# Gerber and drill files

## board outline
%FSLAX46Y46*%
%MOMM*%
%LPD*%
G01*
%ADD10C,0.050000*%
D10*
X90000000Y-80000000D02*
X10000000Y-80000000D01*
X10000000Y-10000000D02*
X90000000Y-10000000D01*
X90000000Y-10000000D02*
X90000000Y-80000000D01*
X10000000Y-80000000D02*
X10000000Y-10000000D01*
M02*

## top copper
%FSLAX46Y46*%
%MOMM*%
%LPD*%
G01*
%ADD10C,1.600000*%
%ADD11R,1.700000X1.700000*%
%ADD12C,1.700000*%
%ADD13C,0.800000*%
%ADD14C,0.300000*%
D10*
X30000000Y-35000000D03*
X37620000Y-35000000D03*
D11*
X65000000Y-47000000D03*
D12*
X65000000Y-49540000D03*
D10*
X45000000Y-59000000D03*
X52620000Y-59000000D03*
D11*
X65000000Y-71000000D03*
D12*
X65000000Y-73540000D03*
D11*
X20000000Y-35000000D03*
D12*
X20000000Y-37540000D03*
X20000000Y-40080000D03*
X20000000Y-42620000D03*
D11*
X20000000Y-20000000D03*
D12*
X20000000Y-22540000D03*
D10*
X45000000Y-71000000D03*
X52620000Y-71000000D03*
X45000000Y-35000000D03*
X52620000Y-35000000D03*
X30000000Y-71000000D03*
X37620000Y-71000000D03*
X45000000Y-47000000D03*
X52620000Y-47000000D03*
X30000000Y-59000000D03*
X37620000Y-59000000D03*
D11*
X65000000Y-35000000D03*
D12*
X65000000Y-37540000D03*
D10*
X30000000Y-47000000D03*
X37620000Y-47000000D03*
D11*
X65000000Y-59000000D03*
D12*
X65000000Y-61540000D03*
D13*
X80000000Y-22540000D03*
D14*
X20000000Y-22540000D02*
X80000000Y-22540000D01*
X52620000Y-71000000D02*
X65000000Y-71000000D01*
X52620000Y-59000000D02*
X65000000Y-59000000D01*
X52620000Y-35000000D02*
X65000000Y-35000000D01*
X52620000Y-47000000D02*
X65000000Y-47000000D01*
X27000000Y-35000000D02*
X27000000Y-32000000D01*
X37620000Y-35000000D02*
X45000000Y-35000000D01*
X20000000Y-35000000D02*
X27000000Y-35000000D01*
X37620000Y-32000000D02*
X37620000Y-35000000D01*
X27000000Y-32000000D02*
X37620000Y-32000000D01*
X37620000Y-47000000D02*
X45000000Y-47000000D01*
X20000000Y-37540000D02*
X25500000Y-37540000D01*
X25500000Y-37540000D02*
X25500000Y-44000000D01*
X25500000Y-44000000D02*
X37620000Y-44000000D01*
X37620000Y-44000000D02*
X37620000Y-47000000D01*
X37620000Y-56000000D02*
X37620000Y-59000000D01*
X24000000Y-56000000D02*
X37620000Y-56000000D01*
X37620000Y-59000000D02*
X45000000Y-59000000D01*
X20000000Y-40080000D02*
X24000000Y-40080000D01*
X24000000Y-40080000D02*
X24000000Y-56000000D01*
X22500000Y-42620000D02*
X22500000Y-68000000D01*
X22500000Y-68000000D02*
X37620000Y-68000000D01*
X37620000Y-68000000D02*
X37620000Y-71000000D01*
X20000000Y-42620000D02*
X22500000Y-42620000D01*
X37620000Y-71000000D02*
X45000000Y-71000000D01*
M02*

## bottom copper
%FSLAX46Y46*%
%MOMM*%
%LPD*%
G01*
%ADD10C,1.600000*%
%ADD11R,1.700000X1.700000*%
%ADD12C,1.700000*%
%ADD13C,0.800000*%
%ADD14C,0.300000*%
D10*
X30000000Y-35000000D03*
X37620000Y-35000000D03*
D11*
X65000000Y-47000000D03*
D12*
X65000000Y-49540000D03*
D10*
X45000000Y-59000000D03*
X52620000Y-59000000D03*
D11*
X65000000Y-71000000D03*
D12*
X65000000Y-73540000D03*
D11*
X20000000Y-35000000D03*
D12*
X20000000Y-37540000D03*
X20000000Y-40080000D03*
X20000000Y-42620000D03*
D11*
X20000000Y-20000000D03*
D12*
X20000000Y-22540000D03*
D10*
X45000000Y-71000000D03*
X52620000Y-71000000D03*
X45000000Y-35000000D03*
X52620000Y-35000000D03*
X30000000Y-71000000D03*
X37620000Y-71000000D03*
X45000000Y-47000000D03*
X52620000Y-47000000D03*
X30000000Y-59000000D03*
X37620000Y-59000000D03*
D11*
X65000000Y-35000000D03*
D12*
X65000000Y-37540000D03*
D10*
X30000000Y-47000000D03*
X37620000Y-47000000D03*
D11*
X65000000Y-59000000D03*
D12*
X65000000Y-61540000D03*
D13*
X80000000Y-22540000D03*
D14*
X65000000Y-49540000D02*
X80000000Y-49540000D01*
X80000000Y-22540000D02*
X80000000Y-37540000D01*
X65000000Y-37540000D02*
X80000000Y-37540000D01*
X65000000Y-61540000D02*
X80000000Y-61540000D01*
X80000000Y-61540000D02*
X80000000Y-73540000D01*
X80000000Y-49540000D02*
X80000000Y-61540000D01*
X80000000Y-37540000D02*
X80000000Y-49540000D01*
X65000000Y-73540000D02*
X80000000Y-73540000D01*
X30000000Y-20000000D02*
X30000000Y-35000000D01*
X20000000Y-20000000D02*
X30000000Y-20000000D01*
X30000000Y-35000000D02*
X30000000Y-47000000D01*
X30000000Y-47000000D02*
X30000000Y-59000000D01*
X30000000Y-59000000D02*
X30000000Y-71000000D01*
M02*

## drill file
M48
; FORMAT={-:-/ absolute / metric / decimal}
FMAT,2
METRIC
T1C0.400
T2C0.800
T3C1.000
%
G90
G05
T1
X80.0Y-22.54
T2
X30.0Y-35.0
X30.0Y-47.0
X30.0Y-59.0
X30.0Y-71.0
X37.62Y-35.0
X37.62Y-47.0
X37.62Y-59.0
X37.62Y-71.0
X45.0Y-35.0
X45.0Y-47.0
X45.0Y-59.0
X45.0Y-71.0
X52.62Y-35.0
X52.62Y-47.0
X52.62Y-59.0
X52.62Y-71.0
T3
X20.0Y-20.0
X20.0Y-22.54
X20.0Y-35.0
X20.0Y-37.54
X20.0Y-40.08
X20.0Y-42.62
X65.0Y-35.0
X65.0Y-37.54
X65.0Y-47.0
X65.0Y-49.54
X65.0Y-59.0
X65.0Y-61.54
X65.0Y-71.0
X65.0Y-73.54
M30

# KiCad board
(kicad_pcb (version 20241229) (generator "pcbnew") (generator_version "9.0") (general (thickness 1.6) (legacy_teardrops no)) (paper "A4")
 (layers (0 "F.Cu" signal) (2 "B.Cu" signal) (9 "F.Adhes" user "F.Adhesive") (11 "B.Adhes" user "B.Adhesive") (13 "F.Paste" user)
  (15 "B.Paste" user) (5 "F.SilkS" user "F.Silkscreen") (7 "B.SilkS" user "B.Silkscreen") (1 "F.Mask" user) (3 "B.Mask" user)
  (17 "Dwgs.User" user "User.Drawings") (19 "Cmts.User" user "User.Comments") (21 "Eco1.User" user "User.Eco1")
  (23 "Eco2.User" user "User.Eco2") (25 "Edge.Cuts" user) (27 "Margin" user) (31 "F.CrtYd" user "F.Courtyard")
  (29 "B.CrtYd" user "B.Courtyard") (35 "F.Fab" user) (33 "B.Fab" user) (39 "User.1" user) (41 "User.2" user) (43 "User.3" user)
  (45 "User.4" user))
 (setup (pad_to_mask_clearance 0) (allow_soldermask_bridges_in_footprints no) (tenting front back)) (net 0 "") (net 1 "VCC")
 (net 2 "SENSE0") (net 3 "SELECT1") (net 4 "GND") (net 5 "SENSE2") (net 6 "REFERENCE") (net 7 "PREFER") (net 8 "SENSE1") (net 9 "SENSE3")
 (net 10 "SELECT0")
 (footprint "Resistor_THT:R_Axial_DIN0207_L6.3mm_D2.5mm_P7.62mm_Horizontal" (layer "F.Cu") (at 30 35)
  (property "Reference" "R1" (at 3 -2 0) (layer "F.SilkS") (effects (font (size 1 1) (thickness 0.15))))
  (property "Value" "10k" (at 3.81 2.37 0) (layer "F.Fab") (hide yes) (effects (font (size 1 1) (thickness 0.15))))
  (pad "1" thru_hole circle (at 0 0) (size 1.6 1.6) (drill 0.8) (layers "*.Cu" "*.Mask") (remove_unused_layers no) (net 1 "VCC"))
  (pad "2" thru_hole circle (at 7.62 0) (size 1.6 1.6) (drill 0.8) (layers "*.Cu" "*.Mask") (remove_unused_layers no) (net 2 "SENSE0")))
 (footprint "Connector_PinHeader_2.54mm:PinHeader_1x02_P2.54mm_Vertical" (layer "F.Cu") (at 65 47)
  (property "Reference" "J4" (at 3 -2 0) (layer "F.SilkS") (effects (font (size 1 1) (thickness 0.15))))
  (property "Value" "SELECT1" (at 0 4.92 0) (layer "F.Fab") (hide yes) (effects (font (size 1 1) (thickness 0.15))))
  (pad "1" thru_hole rect (at 0 0) (size 1.7 1.7) (drill 1) (layers "*.Cu" "*.Mask") (remove_unused_layers no) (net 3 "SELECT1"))
  (pad "2" thru_hole circle (at 0 2.54) (size 1.7 1.7) (drill 1) (layers "*.Cu" "*.Mask") (remove_unused_layers no) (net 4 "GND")))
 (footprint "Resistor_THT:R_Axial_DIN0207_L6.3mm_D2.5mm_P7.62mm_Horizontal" (layer "F.Cu") (at 45 59)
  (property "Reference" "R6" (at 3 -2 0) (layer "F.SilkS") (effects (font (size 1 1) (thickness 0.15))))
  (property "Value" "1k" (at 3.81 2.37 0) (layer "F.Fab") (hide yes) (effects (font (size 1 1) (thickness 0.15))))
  (pad "1" thru_hole circle (at 0 0) (size 1.6 1.6) (drill 0.8) (layers "*.Cu" "*.Mask") (remove_unused_layers no) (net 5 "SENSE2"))
  (pad "2" thru_hole circle (at 7.62 0) (size 1.6 1.6) (drill 0.8) (layers "*.Cu" "*.Mask") (remove_unused_layers no) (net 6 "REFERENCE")))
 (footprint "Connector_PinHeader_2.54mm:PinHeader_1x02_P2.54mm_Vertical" (layer "F.Cu") (at 65 71)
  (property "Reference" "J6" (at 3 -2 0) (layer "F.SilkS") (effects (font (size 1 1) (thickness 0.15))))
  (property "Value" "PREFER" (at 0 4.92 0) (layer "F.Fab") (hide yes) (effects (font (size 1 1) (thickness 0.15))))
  (pad "1" thru_hole rect (at 0 0) (size 1.7 1.7) (drill 1) (layers "*.Cu" "*.Mask") (remove_unused_layers no) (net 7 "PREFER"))
  (pad "2" thru_hole circle (at 0 2.54) (size 1.7 1.7) (drill 1) (layers "*.Cu" "*.Mask") (remove_unused_layers no) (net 4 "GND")))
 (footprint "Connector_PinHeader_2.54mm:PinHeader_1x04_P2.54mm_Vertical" (layer "F.Cu") (at 20 35)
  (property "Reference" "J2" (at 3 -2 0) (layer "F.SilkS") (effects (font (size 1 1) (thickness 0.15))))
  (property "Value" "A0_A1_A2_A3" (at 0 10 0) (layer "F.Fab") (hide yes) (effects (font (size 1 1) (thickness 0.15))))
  (pad "1" thru_hole rect (at 0 0) (size 1.7 1.7) (drill 1) (layers "*.Cu" "*.Mask") (remove_unused_layers no) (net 2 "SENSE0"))
  (pad "2" thru_hole circle (at 0 2.54) (size 1.7 1.7) (drill 1) (layers "*.Cu" "*.Mask") (remove_unused_layers no) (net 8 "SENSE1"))
  (pad "3" thru_hole circle (at 0 5.08) (size 1.7 1.7) (drill 1) (layers "*.Cu" "*.Mask") (remove_unused_layers no) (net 5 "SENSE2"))
  (pad "4" thru_hole circle (at 0 7.62) (size 1.7 1.7) (drill 1) (layers "*.Cu" "*.Mask") (remove_unused_layers no) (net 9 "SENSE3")))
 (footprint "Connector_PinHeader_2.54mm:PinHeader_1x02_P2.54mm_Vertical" (layer "F.Cu") (at 20 20)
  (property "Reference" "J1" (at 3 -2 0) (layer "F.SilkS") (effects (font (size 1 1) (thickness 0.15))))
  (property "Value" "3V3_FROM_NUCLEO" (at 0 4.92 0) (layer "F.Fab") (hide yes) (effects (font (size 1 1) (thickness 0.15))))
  (pad "1" thru_hole rect (at 0 0) (size 1.7 1.7) (drill 1) (layers "*.Cu" "*.Mask") (remove_unused_layers no) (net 1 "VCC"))
  (pad "2" thru_hole circle (at 0 2.54) (size 1.7 1.7) (drill 1) (layers "*.Cu" "*.Mask") (remove_unused_layers no) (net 4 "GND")))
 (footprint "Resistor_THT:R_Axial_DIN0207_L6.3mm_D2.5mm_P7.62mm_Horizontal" (layer "F.Cu") (at 45 71)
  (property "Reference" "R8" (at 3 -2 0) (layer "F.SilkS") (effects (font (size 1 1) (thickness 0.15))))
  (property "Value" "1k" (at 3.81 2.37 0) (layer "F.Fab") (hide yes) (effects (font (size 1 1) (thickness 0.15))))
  (pad "1" thru_hole circle (at 0 0) (size 1.6 1.6) (drill 0.8) (layers "*.Cu" "*.Mask") (remove_unused_layers no) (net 9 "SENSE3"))
  (pad "2" thru_hole circle (at 7.62 0) (size 1.6 1.6) (drill 0.8) (layers "*.Cu" "*.Mask") (remove_unused_layers no) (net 7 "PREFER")))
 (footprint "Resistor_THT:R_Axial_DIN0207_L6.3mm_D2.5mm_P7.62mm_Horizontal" (layer "F.Cu") (at 45 35)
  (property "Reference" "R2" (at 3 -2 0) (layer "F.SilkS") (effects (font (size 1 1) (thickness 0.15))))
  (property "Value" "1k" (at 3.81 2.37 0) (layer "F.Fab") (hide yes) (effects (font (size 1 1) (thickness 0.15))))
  (pad "1" thru_hole circle (at 0 0) (size 1.6 1.6) (drill 0.8) (layers "*.Cu" "*.Mask") (remove_unused_layers no) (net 2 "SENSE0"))
  (pad "2" thru_hole circle (at 7.62 0) (size 1.6 1.6) (drill 0.8) (layers "*.Cu" "*.Mask") (remove_unused_layers no) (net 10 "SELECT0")))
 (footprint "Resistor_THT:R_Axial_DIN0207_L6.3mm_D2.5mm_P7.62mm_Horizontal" (layer "F.Cu") (at 30 71)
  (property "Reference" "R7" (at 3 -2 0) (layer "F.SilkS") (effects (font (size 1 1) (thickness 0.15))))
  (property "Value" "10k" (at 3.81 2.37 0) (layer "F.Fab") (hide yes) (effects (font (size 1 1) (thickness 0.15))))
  (pad "1" thru_hole circle (at 0 0) (size 1.6 1.6) (drill 0.8) (layers "*.Cu" "*.Mask") (remove_unused_layers no) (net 1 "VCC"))
  (pad "2" thru_hole circle (at 7.62 0) (size 1.6 1.6) (drill 0.8) (layers "*.Cu" "*.Mask") (remove_unused_layers no) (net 9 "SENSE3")))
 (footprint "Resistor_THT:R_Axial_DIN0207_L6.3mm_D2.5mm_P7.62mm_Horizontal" (layer "F.Cu") (at 45 47)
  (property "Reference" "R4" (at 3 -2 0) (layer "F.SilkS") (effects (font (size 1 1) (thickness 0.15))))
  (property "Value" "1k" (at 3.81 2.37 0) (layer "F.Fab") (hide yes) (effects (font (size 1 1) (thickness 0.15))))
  (pad "1" thru_hole circle (at 0 0) (size 1.6 1.6) (drill 0.8) (layers "*.Cu" "*.Mask") (remove_unused_layers no) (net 8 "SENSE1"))
  (pad "2" thru_hole circle (at 7.62 0) (size 1.6 1.6) (drill 0.8) (layers "*.Cu" "*.Mask") (remove_unused_layers no) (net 3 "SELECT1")))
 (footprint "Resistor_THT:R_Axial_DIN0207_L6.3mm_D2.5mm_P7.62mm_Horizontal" (layer "F.Cu") (at 30 59)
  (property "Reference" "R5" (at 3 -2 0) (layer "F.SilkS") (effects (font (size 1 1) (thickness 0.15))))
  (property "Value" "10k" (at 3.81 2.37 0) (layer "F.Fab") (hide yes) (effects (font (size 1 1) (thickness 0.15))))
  (pad "1" thru_hole circle (at 0 0) (size 1.6 1.6) (drill 0.8) (layers "*.Cu" "*.Mask") (remove_unused_layers no) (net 1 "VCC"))
  (pad "2" thru_hole circle (at 7.62 0) (size 1.6 1.6) (drill 0.8) (layers "*.Cu" "*.Mask") (remove_unused_layers no) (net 5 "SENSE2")))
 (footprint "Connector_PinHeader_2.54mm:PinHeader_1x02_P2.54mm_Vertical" (layer "F.Cu") (at 65 35)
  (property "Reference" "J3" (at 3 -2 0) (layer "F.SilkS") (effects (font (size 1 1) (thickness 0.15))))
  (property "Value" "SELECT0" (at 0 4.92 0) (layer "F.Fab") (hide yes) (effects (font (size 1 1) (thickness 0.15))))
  (pad "1" thru_hole rect (at 0 0) (size 1.7 1.7) (drill 1) (layers "*.Cu" "*.Mask") (remove_unused_layers no) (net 10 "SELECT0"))
  (pad "2" thru_hole circle (at 0 2.54) (size 1.7 1.7) (drill 1) (layers "*.Cu" "*.Mask") (remove_unused_layers no) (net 4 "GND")))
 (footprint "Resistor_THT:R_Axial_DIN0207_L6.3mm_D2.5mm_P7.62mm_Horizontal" (layer "F.Cu") (at 30 47)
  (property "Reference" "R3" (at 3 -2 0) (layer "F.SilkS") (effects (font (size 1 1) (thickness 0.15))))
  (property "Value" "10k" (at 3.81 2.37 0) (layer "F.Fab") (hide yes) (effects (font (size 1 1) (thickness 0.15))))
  (pad "1" thru_hole circle (at 0 0) (size 1.6 1.6) (drill 0.8) (layers "*.Cu" "*.Mask") (remove_unused_layers no) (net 1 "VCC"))
  (pad "2" thru_hole circle (at 7.62 0) (size 1.6 1.6) (drill 0.8) (layers "*.Cu" "*.Mask") (remove_unused_layers no) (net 8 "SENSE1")))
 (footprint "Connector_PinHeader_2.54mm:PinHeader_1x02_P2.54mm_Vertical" (layer "F.Cu") (at 65 59)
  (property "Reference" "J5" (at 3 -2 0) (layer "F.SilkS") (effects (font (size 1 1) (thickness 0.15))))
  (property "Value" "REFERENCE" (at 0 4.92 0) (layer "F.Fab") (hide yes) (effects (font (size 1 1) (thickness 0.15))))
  (pad "1" thru_hole rect (at 0 0) (size 1.7 1.7) (drill 1) (layers "*.Cu" "*.Mask") (remove_unused_layers no) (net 6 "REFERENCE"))
  (pad "2" thru_hole circle (at 0 2.54) (size 1.7 1.7) (drill 1) (layers "*.Cu" "*.Mask") (remove_unused_layers no) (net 4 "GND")))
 (gr_line (start 90 80) (end 10 80) (stroke (width 0.05) (type default)) (layer "Edge.Cuts"))
 (gr_line (start 10 10) (end 90 10) (stroke (width 0.05) (type default)) (layer "Edge.Cuts"))
 (gr_line (start 90 10) (end 90 80) (stroke (width 0.05) (type default)) (layer "Edge.Cuts"))
 (gr_line (start 10 80) (end 10 10) (stroke (width 0.05) (type default)) (layer "Edge.Cuts"))
 (segment (start 20 22.54) (end 80 22.54) (width 0.3) (layer "F.Cu") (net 4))
 (via (at 80 22.54) (size 0.8) (drill 0.4) (layers "F.Cu" "B.Cu") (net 4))
 (segment (start 65 49.54) (end 80 49.54) (width 0.3) (layer "B.Cu") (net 4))
 (segment (start 80 22.54) (end 80 37.54) (width 0.3) (layer "B.Cu") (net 4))
 (segment (start 65 37.54) (end 80 37.54) (width 0.3) (layer "B.Cu") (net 4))
 (segment (start 65 61.54) (end 80 61.54) (width 0.3) (layer "B.Cu") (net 4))
 (segment (start 80 61.54) (end 80 73.54) (width 0.3) (layer "B.Cu") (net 4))
 (segment (start 80 49.54) (end 80 61.54) (width 0.3) (layer "B.Cu") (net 4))
 (segment (start 80 37.54) (end 80 49.54) (width 0.3) (layer "B.Cu") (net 4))
 (segment (start 65 73.54) (end 80 73.54) (width 0.3) (layer "B.Cu") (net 4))
 (segment (start 52.62 71) (end 65 71) (width 0.3) (layer "F.Cu") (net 7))
 (segment (start 52.62 59) (end 65 59) (width 0.3) (layer "F.Cu") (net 6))
 (segment (start 52.62 35) (end 65 35) (width 0.3) (layer "F.Cu") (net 10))
 (segment (start 52.62 47) (end 65 47) (width 0.3) (layer "F.Cu") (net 3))
 (segment (start 27 35) (end 27 32) (width 0.3) (layer "F.Cu") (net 2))
 (segment (start 37.62 35) (end 45 35) (width 0.3) (layer "F.Cu") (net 2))
 (segment (start 20 35) (end 27 35) (width 0.3) (layer "F.Cu") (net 2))
 (segment (start 37.62 32) (end 37.62 35) (width 0.3) (layer "F.Cu") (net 2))
 (segment (start 27 32) (end 37.62 32) (width 0.3) (layer "F.Cu") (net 2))
 (segment (start 37.62 47) (end 45 47) (width 0.3) (layer "F.Cu") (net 8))
 (segment (start 20 37.54) (end 25.5 37.54) (width 0.3) (layer "F.Cu") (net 8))
 (segment (start 25.5 37.54) (end 25.5 44) (width 0.3) (layer "F.Cu") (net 8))
 (segment (start 25.5 44) (end 37.62 44) (width 0.3) (layer "F.Cu") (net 8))
 (segment (start 37.62 44) (end 37.62 47) (width 0.3) (layer "F.Cu") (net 8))
 (segment (start 37.62 56) (end 37.62 59) (width 0.3) (layer "F.Cu") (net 5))
 (segment (start 24 56) (end 37.62 56) (width 0.3) (layer "F.Cu") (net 5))
 (segment (start 37.62 59) (end 45 59) (width 0.3) (layer "F.Cu") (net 5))
 (segment (start 20 40.08) (end 24 40.08) (width 0.3) (layer "F.Cu") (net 5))
 (segment (start 24 40.08) (end 24 56) (width 0.3) (layer "F.Cu") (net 5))
 (segment (start 22.5 42.62) (end 22.5 68) (width 0.3) (layer "F.Cu") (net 9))
 (segment (start 22.5 68) (end 37.62 68) (width 0.3) (layer "F.Cu") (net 9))
 (segment (start 37.62 68) (end 37.62 71) (width 0.3) (layer "F.Cu") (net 9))
 (segment (start 20 42.62) (end 22.5 42.62) (width 0.3) (layer "F.Cu") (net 9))
 (segment (start 37.62 71) (end 45 71) (width 0.3) (layer "F.Cu") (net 9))
 (segment (start 30 20) (end 30 35) (width 0.3) (layer "B.Cu") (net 1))
 (segment (start 20 20) (end 30 20) (width 0.3) (layer "B.Cu") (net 1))
 (segment (start 30 35) (end 30 47) (width 0.3) (layer "B.Cu") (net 1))
 (segment (start 30 47) (end 30 59) (width 0.3) (layer "B.Cu") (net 1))
 (segment (start 30 59) (end 30 71) (width 0.3) (layer "B.Cu") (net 1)))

